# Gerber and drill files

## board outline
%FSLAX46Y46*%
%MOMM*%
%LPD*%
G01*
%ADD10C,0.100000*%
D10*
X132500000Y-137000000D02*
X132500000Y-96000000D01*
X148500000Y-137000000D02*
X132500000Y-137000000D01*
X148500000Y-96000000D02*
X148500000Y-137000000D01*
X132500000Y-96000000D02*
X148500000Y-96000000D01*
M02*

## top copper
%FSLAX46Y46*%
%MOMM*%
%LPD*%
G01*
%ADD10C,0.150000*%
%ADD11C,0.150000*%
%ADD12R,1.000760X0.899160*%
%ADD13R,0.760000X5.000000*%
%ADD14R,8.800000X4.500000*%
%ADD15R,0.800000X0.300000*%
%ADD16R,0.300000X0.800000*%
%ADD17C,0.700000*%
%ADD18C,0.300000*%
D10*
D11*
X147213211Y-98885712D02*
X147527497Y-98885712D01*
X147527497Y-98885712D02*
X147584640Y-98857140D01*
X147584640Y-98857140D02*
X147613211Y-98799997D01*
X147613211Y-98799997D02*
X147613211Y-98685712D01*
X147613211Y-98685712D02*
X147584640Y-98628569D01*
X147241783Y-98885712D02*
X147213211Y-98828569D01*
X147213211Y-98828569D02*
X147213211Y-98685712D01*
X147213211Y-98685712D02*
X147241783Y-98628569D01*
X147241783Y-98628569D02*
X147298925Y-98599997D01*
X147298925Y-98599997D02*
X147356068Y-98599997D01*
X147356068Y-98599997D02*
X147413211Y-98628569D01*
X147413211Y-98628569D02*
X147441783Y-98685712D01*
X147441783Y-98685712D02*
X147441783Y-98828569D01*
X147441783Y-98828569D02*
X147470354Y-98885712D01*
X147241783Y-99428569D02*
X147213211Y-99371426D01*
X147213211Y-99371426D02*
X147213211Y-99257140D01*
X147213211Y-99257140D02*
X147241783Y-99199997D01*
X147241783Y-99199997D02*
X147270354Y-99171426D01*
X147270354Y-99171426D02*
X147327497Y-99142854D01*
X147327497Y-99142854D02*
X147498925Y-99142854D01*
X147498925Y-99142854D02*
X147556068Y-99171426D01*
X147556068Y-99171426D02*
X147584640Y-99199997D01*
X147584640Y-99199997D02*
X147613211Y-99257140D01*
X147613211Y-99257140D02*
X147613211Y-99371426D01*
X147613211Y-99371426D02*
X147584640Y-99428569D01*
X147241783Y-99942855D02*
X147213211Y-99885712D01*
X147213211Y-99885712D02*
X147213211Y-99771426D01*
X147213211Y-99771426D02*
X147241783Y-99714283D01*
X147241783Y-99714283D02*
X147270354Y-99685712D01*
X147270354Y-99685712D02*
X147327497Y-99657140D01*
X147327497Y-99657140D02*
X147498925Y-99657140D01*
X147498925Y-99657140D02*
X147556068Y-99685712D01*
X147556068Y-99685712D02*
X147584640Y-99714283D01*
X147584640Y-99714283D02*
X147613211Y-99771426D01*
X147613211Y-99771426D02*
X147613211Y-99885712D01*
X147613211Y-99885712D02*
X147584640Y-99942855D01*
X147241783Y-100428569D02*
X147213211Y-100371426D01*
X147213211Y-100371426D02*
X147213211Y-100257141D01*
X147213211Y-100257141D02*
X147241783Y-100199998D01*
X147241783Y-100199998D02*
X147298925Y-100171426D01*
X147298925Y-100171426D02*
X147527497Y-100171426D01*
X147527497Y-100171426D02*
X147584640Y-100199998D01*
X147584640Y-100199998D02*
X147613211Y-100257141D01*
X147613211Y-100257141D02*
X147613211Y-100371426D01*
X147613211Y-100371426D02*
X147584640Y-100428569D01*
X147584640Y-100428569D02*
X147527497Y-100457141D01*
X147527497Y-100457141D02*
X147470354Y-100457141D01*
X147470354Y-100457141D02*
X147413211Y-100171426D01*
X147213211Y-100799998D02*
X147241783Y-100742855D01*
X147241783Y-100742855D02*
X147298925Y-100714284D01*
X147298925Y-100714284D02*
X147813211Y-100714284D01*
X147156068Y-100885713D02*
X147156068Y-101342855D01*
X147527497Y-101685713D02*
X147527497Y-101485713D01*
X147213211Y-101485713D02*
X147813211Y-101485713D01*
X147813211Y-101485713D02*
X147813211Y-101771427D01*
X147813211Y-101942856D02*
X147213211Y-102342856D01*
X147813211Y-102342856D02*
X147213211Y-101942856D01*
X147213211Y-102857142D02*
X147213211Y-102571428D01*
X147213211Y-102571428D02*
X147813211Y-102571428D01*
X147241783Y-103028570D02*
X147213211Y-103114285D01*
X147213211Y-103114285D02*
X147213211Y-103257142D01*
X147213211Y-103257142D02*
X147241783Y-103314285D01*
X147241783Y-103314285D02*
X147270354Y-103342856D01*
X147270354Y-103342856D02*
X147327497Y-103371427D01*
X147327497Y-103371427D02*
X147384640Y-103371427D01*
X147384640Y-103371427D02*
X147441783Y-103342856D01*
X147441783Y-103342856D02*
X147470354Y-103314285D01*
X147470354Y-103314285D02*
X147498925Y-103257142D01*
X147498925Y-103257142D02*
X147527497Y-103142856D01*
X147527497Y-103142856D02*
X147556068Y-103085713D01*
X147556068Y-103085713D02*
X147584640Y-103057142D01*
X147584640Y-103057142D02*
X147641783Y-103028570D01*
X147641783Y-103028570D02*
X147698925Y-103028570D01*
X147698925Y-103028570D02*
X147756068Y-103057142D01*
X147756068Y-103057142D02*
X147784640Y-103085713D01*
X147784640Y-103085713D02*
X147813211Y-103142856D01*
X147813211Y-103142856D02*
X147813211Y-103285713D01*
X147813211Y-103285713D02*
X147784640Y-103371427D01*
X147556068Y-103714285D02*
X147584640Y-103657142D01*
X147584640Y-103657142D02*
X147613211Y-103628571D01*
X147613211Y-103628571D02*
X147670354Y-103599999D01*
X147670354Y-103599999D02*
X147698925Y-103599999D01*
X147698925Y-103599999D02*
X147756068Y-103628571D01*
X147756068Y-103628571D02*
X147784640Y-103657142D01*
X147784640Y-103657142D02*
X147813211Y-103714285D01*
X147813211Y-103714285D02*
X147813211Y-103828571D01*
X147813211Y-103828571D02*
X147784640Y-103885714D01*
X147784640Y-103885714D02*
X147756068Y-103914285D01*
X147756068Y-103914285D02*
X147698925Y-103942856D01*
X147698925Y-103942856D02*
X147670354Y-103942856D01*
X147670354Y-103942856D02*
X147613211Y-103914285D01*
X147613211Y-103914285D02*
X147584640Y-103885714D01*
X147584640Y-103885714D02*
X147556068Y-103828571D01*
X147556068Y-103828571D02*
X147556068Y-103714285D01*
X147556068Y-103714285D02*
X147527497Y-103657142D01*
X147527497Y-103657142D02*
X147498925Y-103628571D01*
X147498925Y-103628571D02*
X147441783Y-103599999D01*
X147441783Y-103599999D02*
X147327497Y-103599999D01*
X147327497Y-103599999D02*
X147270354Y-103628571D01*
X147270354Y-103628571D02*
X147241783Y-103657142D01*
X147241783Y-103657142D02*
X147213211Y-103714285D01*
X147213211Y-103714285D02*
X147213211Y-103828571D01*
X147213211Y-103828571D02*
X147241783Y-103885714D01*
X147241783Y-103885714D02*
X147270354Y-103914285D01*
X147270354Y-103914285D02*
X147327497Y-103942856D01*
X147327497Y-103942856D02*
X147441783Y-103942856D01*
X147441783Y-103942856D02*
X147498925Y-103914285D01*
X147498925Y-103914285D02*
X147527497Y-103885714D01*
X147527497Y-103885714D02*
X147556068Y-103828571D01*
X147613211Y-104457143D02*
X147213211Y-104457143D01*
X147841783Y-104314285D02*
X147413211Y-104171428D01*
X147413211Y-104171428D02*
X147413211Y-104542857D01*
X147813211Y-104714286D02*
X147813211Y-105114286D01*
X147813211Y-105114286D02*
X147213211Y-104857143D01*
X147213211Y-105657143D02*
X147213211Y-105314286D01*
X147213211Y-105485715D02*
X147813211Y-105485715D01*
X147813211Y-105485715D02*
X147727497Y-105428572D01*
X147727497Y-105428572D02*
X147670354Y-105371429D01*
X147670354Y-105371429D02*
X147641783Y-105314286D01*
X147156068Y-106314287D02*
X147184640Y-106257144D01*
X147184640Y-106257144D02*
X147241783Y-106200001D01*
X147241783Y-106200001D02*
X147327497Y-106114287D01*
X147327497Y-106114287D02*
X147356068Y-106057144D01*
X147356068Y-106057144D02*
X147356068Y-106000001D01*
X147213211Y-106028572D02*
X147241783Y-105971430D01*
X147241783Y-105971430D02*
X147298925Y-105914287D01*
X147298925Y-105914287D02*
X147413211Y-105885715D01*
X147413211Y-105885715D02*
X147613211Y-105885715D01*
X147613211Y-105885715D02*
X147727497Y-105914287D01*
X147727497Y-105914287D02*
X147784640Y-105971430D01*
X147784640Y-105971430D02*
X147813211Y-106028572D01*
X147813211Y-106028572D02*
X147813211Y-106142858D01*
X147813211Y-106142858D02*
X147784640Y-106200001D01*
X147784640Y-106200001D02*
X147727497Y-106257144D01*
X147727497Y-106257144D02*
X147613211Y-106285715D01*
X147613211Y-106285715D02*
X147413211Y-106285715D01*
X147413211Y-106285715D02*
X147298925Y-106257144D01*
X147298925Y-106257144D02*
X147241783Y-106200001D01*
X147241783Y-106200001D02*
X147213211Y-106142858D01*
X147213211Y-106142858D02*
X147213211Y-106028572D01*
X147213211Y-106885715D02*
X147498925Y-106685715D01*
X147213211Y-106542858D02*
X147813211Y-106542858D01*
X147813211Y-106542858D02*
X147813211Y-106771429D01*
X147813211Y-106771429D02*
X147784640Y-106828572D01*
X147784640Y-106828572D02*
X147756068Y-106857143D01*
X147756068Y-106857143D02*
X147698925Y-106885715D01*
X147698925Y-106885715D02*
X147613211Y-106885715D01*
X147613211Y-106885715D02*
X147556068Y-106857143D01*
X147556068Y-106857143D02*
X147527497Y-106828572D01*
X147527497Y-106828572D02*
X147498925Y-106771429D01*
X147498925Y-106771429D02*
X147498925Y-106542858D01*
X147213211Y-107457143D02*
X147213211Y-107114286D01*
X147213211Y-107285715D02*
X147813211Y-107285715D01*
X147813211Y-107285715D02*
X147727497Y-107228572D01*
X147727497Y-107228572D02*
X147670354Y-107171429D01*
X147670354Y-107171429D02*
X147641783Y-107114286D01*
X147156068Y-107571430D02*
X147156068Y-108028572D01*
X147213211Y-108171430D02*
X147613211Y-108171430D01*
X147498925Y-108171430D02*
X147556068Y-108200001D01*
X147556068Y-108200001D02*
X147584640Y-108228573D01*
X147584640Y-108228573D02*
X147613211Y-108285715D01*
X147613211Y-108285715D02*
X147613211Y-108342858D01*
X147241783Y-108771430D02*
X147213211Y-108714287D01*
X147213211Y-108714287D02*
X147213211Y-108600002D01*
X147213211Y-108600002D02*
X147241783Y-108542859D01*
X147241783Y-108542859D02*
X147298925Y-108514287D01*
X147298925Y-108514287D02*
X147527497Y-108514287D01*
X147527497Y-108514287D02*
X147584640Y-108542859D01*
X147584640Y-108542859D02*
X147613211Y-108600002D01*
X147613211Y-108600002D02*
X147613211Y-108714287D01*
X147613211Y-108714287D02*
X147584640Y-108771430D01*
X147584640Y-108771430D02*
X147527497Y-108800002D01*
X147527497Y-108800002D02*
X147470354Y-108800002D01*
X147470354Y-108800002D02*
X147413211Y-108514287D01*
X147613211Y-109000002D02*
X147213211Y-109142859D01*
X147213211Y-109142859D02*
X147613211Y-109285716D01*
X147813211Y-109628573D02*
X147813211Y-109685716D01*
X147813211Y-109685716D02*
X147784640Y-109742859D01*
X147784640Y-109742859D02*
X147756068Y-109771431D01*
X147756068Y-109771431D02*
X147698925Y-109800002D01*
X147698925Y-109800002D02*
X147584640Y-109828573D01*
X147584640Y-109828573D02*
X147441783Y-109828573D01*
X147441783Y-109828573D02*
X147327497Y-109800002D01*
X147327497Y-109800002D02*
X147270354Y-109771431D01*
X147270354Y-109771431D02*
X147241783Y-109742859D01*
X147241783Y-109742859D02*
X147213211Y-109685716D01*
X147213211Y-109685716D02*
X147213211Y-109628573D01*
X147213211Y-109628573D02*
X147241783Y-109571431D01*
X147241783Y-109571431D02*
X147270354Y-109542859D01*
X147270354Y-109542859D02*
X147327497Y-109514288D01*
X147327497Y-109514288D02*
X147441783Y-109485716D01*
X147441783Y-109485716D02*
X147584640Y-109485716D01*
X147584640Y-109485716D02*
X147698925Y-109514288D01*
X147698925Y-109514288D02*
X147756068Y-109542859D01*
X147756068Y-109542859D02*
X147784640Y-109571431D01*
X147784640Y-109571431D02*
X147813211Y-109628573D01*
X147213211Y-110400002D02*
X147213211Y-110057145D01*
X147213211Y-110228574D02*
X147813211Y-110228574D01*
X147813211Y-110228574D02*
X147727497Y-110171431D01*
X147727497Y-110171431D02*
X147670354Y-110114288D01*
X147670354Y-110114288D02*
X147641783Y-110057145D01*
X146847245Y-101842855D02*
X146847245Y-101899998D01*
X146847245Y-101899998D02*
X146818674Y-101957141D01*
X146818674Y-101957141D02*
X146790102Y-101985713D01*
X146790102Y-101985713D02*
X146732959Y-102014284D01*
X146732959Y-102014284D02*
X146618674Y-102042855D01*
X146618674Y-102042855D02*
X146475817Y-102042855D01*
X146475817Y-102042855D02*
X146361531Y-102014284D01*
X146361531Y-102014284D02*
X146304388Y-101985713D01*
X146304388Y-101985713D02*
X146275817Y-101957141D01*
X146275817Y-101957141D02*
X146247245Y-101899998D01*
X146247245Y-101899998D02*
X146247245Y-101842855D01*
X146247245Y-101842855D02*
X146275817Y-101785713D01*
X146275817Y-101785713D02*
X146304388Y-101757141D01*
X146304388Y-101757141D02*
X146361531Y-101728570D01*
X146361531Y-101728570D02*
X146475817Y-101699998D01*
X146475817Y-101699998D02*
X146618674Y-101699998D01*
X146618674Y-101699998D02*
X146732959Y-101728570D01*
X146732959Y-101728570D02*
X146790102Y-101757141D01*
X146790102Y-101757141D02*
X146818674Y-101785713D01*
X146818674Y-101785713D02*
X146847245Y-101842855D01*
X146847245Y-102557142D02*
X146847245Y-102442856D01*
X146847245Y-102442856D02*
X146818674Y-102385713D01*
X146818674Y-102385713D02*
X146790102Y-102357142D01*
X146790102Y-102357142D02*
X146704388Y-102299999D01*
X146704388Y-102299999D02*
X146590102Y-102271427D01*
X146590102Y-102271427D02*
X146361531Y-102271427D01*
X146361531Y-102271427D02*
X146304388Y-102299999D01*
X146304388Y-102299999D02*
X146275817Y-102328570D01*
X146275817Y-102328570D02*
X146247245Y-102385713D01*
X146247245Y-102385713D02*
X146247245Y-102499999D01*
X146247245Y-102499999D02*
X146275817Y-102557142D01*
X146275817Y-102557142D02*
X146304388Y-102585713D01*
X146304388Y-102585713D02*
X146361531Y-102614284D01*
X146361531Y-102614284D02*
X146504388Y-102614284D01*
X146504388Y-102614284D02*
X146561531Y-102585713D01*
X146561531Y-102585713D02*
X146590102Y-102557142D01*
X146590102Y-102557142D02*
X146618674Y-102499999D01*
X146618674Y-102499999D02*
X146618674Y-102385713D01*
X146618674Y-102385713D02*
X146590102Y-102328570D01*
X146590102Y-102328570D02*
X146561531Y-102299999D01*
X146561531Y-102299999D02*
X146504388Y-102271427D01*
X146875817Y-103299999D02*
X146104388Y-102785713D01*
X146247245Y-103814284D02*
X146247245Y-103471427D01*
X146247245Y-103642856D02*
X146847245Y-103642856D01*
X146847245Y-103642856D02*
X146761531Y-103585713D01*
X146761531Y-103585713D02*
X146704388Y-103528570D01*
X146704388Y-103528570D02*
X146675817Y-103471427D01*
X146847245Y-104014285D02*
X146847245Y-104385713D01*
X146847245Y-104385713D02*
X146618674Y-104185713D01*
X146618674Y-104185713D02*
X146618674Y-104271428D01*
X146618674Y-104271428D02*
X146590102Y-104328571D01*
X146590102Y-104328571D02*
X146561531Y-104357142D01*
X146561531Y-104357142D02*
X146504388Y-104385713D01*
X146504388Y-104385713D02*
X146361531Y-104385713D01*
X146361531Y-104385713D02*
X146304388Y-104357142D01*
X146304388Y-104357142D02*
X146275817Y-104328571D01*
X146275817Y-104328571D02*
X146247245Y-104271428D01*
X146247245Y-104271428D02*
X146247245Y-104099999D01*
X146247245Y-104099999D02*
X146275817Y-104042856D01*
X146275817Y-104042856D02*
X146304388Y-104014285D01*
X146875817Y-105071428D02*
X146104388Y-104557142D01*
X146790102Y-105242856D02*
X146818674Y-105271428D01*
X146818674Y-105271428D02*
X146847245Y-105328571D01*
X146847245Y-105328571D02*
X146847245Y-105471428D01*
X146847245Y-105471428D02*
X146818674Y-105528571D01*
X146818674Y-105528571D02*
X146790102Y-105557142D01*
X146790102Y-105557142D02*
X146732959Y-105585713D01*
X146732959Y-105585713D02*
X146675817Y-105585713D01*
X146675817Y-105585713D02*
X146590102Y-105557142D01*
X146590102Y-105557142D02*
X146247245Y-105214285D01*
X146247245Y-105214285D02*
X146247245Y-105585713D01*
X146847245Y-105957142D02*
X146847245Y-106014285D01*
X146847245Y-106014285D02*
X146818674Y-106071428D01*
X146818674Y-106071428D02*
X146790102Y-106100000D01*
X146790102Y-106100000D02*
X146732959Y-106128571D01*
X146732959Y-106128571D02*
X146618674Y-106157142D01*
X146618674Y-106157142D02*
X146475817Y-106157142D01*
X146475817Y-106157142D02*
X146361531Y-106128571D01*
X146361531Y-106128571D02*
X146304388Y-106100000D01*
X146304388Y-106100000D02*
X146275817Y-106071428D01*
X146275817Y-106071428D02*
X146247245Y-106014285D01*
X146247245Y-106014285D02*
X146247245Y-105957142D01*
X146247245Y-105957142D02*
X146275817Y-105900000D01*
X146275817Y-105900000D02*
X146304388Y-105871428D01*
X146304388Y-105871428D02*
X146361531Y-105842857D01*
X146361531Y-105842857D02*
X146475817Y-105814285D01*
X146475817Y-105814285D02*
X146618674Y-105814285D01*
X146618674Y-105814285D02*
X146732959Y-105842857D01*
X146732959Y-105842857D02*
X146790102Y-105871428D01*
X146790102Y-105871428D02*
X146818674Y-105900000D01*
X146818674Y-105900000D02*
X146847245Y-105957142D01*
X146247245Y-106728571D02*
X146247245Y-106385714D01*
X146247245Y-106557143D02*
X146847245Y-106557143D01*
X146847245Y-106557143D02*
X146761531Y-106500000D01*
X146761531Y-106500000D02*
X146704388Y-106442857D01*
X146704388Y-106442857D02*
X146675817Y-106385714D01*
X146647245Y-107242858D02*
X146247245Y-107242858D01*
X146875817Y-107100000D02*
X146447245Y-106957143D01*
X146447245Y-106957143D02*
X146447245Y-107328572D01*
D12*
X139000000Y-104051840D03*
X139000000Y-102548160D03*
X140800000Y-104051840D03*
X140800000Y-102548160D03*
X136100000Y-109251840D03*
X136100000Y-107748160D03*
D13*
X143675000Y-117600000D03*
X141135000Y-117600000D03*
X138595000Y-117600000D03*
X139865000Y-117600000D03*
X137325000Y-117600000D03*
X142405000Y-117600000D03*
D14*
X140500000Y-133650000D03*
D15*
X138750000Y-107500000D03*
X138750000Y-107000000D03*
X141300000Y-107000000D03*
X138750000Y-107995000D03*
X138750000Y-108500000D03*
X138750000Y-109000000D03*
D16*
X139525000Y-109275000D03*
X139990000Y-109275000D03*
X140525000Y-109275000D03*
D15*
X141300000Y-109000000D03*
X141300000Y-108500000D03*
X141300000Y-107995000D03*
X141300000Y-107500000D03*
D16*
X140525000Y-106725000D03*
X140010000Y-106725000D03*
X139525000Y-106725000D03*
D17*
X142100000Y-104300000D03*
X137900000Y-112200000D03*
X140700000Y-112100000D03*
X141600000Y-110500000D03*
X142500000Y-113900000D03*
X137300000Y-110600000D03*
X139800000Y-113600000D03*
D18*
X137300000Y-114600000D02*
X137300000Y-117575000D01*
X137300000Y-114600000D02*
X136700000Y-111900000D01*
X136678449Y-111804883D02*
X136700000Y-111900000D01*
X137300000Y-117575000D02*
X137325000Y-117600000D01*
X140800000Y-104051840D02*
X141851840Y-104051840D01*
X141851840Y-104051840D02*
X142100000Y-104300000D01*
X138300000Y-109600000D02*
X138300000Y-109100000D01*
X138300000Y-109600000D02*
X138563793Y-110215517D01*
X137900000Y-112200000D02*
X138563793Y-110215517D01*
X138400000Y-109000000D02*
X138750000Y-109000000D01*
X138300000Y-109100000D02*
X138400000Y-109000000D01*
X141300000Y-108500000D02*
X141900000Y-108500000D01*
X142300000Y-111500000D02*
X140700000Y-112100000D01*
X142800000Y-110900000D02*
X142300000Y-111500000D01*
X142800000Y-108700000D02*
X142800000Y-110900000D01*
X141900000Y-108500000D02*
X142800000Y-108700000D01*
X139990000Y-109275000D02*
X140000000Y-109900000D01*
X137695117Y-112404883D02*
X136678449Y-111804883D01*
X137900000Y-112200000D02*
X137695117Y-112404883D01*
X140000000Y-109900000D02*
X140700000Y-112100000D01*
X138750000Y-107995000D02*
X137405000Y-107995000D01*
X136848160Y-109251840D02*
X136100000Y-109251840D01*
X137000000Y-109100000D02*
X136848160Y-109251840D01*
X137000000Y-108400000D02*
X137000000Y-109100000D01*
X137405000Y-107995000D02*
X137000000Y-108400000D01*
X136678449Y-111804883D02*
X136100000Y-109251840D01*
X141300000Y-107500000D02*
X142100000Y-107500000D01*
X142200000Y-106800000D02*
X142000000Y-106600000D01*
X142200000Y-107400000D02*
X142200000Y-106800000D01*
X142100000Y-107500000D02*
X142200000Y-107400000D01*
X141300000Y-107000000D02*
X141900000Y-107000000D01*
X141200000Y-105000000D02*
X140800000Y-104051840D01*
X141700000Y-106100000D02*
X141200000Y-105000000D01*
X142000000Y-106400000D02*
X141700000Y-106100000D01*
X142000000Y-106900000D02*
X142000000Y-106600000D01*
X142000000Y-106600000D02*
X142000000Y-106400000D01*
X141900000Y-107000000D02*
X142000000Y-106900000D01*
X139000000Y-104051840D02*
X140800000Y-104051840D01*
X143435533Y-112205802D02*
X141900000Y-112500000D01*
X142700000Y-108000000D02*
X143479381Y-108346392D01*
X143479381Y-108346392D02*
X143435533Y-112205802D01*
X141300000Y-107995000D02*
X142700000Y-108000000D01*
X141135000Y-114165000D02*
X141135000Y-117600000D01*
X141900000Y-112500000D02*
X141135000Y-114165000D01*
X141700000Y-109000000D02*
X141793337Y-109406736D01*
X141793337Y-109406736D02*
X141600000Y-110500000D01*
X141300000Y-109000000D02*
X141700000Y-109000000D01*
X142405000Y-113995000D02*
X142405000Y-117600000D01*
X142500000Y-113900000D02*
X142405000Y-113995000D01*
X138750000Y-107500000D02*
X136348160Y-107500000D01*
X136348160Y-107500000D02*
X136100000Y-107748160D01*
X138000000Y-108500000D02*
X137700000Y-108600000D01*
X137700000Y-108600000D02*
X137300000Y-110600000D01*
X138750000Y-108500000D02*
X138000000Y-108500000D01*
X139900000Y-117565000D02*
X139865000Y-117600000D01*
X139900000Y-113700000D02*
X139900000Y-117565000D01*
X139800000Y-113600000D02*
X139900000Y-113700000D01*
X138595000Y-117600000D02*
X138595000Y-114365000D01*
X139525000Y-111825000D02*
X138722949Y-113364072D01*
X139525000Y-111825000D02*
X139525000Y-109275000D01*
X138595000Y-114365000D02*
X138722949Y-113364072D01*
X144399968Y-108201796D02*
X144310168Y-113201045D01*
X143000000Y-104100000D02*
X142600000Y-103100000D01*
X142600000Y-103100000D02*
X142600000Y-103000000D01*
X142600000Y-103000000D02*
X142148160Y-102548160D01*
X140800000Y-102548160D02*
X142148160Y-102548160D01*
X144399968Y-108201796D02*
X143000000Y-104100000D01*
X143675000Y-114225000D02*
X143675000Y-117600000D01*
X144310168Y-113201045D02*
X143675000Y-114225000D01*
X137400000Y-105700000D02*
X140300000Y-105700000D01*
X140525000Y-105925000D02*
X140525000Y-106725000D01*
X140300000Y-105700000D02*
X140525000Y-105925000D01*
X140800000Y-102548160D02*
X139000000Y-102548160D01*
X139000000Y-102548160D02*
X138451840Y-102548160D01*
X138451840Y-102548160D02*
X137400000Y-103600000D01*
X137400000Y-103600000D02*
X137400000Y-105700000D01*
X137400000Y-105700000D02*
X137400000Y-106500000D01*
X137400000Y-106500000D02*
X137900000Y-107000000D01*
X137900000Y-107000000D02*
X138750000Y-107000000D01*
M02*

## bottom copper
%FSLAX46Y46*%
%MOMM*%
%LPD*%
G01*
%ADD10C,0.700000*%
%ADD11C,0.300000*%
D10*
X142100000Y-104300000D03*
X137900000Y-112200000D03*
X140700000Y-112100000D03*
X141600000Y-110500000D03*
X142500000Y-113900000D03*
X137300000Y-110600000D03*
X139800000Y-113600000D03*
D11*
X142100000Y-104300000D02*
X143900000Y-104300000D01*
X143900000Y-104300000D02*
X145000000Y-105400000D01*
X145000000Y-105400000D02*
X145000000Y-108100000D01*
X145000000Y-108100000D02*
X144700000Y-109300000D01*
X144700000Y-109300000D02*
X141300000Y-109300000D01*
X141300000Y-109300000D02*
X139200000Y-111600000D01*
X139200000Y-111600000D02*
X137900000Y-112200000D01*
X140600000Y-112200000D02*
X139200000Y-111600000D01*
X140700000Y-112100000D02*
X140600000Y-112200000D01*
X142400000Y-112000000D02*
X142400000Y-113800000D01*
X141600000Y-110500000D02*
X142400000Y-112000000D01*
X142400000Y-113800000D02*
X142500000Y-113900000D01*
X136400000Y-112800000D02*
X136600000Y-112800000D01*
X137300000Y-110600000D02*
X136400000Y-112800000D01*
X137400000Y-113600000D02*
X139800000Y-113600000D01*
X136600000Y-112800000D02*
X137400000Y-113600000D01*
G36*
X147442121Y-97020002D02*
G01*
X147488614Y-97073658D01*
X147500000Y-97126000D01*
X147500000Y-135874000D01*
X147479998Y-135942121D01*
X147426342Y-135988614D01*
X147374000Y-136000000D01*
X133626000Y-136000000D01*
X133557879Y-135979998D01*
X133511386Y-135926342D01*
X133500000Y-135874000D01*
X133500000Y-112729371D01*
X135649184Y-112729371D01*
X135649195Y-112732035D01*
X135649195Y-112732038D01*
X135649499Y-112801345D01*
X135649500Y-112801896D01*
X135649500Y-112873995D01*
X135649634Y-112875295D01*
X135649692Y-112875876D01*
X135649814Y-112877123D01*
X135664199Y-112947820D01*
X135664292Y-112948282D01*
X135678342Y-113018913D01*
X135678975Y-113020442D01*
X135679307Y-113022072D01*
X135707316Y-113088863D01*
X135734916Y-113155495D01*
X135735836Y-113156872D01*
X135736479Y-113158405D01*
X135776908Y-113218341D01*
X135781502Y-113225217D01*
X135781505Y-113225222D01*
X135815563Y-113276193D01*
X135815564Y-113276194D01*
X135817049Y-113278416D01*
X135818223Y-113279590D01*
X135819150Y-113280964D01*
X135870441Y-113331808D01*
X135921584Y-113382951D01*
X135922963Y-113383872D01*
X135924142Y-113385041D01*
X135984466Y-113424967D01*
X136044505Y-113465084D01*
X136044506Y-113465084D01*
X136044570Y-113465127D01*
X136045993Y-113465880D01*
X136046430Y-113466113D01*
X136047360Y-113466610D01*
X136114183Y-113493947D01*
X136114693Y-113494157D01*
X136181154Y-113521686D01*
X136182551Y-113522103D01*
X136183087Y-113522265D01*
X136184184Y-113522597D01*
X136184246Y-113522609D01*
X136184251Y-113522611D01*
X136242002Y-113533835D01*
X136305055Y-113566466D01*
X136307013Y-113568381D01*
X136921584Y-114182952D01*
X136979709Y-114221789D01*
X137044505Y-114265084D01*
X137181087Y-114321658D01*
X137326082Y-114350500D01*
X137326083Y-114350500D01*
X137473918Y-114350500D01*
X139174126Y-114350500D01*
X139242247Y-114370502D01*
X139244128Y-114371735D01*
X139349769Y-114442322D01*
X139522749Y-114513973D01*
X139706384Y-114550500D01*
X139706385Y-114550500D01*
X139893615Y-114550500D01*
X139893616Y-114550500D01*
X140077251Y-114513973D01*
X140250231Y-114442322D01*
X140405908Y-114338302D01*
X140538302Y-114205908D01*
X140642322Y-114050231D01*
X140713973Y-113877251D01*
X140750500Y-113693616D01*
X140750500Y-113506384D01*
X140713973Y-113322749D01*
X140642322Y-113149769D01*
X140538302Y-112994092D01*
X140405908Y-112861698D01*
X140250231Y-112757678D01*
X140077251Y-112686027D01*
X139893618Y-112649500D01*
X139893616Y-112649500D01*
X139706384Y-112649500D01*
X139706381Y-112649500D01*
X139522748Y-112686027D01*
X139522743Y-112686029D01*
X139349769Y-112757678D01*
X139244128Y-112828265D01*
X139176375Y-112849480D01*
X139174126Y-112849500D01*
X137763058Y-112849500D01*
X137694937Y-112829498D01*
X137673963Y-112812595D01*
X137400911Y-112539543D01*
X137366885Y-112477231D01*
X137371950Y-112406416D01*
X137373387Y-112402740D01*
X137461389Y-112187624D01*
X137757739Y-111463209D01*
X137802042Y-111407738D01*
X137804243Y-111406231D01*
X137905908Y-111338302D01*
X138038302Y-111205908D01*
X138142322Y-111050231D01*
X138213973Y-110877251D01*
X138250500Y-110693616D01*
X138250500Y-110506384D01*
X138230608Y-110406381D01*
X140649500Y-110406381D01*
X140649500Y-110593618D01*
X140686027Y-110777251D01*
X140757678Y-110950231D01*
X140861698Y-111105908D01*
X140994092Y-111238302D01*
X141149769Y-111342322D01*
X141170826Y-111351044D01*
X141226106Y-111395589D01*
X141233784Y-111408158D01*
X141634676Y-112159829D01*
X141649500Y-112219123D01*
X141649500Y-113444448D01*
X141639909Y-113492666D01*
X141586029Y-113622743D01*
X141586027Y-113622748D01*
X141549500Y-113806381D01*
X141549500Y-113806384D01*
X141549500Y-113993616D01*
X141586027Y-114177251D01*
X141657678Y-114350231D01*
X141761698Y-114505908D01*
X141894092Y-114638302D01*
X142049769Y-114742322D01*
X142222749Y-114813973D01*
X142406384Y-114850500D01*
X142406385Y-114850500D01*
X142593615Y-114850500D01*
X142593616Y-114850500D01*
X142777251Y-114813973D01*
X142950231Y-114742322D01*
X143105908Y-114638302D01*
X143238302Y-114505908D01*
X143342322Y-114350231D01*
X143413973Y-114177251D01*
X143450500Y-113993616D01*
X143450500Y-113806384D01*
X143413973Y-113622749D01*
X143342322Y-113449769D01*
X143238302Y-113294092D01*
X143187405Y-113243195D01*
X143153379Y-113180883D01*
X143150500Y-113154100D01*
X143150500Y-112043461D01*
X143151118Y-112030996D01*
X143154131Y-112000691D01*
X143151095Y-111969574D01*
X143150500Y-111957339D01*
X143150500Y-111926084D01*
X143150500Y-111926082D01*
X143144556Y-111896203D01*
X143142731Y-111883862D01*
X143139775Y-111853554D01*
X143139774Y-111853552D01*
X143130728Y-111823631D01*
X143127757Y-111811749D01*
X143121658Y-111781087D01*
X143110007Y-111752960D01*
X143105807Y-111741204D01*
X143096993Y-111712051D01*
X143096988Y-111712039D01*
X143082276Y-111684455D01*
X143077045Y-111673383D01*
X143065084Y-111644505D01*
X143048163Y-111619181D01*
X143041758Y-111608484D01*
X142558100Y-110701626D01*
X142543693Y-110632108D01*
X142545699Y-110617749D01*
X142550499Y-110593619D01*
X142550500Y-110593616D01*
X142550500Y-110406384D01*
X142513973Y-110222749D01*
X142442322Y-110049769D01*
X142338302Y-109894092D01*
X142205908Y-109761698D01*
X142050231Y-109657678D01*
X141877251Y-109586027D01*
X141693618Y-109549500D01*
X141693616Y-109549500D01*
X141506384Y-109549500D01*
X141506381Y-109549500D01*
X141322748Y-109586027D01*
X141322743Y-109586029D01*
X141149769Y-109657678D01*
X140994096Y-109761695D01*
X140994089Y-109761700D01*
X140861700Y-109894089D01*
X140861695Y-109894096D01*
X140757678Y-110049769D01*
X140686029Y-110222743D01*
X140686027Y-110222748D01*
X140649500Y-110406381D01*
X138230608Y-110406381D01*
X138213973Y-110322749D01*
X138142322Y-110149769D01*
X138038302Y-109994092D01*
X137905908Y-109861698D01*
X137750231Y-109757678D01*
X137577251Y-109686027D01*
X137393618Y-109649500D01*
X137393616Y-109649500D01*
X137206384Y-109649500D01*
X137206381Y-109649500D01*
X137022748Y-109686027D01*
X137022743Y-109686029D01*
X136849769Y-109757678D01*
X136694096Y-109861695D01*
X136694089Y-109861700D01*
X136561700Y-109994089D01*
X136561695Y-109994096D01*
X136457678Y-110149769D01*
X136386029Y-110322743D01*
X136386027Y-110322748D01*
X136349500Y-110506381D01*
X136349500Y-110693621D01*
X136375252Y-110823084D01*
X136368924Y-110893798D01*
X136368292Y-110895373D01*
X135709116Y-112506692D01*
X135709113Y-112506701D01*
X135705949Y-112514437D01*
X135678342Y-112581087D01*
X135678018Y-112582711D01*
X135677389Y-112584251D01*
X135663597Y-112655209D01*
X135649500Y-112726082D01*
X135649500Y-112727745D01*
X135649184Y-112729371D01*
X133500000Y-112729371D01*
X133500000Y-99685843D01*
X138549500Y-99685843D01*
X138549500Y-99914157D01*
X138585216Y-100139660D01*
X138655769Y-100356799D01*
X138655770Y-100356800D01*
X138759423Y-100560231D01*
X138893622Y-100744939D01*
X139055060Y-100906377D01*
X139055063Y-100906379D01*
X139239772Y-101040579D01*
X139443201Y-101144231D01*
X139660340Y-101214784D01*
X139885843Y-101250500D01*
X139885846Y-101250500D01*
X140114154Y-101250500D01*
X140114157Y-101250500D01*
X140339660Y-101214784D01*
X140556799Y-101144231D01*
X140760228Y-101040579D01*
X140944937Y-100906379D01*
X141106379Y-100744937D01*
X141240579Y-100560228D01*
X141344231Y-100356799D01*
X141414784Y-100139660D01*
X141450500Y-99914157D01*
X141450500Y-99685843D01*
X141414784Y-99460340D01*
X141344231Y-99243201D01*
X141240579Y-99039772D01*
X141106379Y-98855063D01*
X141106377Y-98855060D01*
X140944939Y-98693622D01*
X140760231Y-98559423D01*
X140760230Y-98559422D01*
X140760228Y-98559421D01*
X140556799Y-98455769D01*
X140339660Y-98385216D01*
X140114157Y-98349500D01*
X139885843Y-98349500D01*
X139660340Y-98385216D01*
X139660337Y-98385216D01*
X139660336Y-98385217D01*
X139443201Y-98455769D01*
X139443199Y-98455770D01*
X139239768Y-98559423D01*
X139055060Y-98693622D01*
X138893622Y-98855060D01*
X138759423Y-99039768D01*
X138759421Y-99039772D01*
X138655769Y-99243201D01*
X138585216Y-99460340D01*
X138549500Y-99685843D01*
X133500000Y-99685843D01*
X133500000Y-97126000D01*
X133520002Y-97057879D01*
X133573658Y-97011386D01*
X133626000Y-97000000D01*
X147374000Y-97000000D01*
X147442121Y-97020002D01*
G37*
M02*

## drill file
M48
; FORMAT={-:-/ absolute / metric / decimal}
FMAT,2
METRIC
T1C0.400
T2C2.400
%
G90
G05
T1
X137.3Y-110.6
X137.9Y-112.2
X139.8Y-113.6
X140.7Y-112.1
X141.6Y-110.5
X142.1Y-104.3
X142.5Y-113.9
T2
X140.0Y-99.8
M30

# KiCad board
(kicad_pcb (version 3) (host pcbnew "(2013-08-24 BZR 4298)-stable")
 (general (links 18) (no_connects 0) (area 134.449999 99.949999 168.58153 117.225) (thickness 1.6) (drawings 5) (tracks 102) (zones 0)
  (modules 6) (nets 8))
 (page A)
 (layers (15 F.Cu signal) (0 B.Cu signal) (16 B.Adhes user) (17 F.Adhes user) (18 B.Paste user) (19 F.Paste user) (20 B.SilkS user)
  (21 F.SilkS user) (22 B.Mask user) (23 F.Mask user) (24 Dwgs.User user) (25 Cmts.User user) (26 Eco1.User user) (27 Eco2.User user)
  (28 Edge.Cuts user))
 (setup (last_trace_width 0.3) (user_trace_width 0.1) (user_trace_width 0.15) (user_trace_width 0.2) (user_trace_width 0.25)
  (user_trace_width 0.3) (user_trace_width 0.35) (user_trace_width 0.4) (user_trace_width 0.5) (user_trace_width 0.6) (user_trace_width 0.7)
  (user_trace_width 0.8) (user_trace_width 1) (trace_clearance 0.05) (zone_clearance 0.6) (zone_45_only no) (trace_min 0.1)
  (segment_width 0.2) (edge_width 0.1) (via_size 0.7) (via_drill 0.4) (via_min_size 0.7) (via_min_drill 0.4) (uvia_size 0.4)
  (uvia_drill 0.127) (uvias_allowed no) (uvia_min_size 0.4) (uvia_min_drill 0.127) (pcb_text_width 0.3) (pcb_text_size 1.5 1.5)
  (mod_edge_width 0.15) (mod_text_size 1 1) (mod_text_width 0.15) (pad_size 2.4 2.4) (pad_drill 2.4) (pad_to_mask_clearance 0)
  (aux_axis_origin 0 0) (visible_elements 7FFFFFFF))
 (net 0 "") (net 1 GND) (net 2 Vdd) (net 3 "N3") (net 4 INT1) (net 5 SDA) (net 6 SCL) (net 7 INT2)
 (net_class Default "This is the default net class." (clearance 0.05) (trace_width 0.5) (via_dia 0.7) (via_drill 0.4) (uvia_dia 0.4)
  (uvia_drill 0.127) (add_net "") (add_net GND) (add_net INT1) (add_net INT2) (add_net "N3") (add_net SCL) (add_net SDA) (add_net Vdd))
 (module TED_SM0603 (layer F.Cu) (at 139 103.3 270)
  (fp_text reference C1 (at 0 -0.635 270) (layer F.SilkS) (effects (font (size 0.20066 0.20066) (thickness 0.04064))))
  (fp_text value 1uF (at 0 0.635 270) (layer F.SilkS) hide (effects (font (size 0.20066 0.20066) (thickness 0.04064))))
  (pad 2 smd rect (at 0.75184 0 270) (size 0.89916 1.00076) (layers F.Cu F.Paste F.Mask) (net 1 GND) (clearance 0.1))
  (pad 1 smd rect (at -0.75184 0 270) (size 0.89916 1.00076) (layers F.Cu F.Paste F.Mask) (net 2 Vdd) (clearance 0.1)))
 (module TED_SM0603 (layer F.Cu) (at 140.8 103.3 270)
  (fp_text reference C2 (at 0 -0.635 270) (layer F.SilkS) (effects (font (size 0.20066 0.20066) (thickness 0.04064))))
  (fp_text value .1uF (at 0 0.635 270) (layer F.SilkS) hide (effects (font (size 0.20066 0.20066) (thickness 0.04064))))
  (pad 2 smd rect (at 0.75184 0 270) (size 0.89916 1.00076) (layers F.Cu F.Paste F.Mask) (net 1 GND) (clearance 0.1))
  (pad 1 smd rect (at -0.75184 0 270) (size 0.89916 1.00076) (layers F.Cu F.Paste F.Mask) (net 2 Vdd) (clearance 0.1)))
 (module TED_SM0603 (layer F.Cu) (at 136.1 108.5 270)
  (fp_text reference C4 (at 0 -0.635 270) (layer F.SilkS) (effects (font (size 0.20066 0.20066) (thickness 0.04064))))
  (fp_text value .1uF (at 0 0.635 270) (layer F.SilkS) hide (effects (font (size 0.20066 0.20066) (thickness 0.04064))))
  (pad 2 smd rect (at 0.75184 0 270) (size 0.89916 1.00076) (layers F.Cu F.Paste F.Mask) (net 1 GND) (clearance 0.1))
  (pad 1 smd rect (at -0.75184 0 270) (size 0.89916 1.00076) (layers F.Cu F.Paste F.Mask) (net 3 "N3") (clearance 0.1)))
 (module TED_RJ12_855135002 (layer F.Cu) (at 140.5 125.5 180)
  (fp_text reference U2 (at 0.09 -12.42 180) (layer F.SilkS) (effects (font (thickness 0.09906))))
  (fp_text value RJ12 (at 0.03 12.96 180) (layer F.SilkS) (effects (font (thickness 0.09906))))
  (pad 6 smd rect (at -3.175 7.9 180) (size 0.76 5) (layers F.Cu F.Paste F.Mask) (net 2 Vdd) (clearance 0.2))
  (pad 4 smd rect (at -0.635 7.9 180) (size 0.76 5) (layers F.Cu F.Paste F.Mask) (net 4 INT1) (clearance 0.2))
  (pad 2 smd rect (at 1.905 7.9 180) (size 0.76 5) (layers F.Cu F.Paste F.Mask) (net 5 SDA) (clearance 0.2))
  (pad 3 smd rect (at 0.635 7.9 180) (size 0.76 5) (layers F.Cu F.Paste F.Mask) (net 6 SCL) (clearance 0.2))
  (pad 1 smd rect (at 3.175 7.9 180) (size 0.76 5) (layers F.Cu F.Paste F.Mask) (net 1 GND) (clearance 0.2))
  (pad 5 smd rect (at -1.905 7.9 180) (size 0.76 5) (layers F.Cu F.Paste F.Mask) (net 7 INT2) (clearance 0.2))
  (pad PAD smd rect (at 0 -8.15 180) (size 8.8 4.5) (layers F.Cu F.Paste F.Mask)))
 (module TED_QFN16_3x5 (layer F.Cu) (at 140.025 108) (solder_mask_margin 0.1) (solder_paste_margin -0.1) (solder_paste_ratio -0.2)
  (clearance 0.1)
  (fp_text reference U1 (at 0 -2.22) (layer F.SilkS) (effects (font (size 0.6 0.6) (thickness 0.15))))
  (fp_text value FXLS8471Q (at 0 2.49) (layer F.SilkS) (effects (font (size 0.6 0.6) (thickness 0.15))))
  (pad 2 smd rect (at -1.275 -0.5) (size 0.8 0.3) (layers F.Cu F.Paste F.Mask) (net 3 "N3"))
  (pad 1 smd rect (at -1.275 -1) (size 0.8 0.3) (layers F.Cu F.Paste F.Mask) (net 2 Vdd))
  (pad 13 smd rect (at 1.275 -1) (size 0.8 0.3) (layers F.Cu F.Paste F.Mask) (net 1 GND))
  (pad 3 smd rect (at -1.275 -0.005) (size 0.8 0.3) (layers F.Cu F.Paste F.Mask) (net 1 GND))
  (pad 4 smd rect (at -1.275 0.5) (size 0.8 0.3) (layers F.Cu F.Paste F.Mask) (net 6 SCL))
  (pad 5 smd rect (at -1.275 1) (size 0.8 0.3) (layers F.Cu F.Paste F.Mask) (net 1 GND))
  (pad 6 smd rect (at -0.5 1.275) (size 0.3 0.8) (layers F.Cu F.Paste F.Mask) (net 5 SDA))
  (pad 7 smd rect (at -0.035 1.275) (size 0.3 0.8) (layers F.Cu F.Paste F.Mask) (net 1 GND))
  (pad 8 smd rect (at 0.5 1.275) (size 0.3 0.8) (layers F.Cu F.Paste F.Mask))
  (pad 9 smd rect (at 1.275 1) (size 0.8 0.3) (layers F.Cu F.Paste F.Mask) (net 7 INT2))
  (pad 10 smd rect (at 1.275 0.5) (size 0.8 0.3) (layers F.Cu F.Paste F.Mask) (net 1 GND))
  (pad 11 smd rect (at 1.275 -0.005) (size 0.8 0.3) (layers F.Cu F.Paste F.Mask) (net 4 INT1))
  (pad 12 smd rect (at 1.275 -0.5) (size 0.8 0.3) (layers F.Cu F.Paste F.Mask) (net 1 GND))
  (pad 14 smd rect (at 0.5 -1.275) (size 0.3 0.8) (layers F.Cu F.Paste F.Mask) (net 2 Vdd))
  (pad 15 smd rect (at -0.015 -1.275) (size 0.3 0.8) (layers F.Cu F.Paste F.Mask))
  (pad 16 smd rect (at -0.5 -1.275) (size 0.3 0.8) (layers F.Cu F.Paste F.Mask)))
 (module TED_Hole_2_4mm (layer F.Cu) (at 140 99.8)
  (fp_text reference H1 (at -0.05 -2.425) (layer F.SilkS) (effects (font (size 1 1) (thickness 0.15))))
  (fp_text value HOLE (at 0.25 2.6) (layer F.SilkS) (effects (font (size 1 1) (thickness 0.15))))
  (pad "" np_thru_hole circle (at 0 0) (size 2.4 2.4) (drill 2.4) (layers *.Cu *.Mask F.SilkS)))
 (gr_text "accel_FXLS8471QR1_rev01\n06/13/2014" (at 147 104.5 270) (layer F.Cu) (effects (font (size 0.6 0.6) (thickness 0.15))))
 (gr_line (start 132.5 137) (end 132.5 96) (angle 90) (layer Edge.Cuts) (width 0.1))
 (gr_line (start 148.5 137) (end 132.5 137) (angle 90) (layer Edge.Cuts) (width 0.1))
 (gr_line (start 148.5 96) (end 148.5 137) (angle 90) (layer Edge.Cuts) (width 0.1))
 (gr_line (start 132.5 96) (end 148.5 96) (angle 90) (layer Edge.Cuts) (width 0.1))
 (segment (start 137.3 114.6) (end 137.3 117.575) (width 0.3) (layer F.Cu) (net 1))
 (segment (start 137.3 114.6) (end 136.7 111.9) (width 0.3) (layer F.Cu) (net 1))
 (segment (start 136.678449 111.804883) (end 136.7 111.9) (width 0.3) (layer F.Cu) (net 1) (status 20))
 (segment (start 137.3 117.575) (end 137.325 117.6) (width 0.3) (layer F.Cu) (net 1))
 (segment (start 140.8 104.05184) (end 141.85184 104.05184) (width 0.3) (layer F.Cu) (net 1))
 (segment (start 141.85184 104.05184) (end 142.1 104.3) (width 0.3) (layer F.Cu) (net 1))
 (via (at 142.1 104.3) (size 0.7) (layers F.Cu B.Cu) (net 1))
 (segment (start 142.1 104.3) (end 143.9 104.3) (width 0.3) (layer B.Cu) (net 1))
 (segment (start 143.9 104.3) (end 145 105.4) (width 0.3) (layer B.Cu) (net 1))
 (segment (start 145 105.4) (end 145 108.1) (width 0.3) (layer B.Cu) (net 1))
 (segment (start 145 108.1) (end 144.7 109.3) (width 0.3) (layer B.Cu) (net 1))
 (segment (start 144.7 109.3) (end 141.3 109.3) (width 0.3) (layer B.Cu) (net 1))
 (segment (start 141.3 109.3) (end 139.2 111.6) (width 0.3) (layer B.Cu) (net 1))
 (segment (start 138.3 109.6) (end 138.3 109.1) (width 0.3) (layer F.Cu) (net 1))
 (segment (start 138.3 109.6) (end 138.563793 110.215517) (width 0.3) (layer F.Cu) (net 1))
 (segment (start 137.9 112.2) (end 138.563793 110.215517) (width 0.3) (layer F.Cu) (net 1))
 (segment (start 138.4 109) (end 138.75 109) (width 0.3) (layer F.Cu) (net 1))
 (segment (start 138.3 109.1) (end 138.4 109) (width 0.3) (layer F.Cu) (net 1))
 (segment (start 141.3 108.5) (end 141.9 108.5) (width 0.3) (layer F.Cu) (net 1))
 (segment (start 142.3 111.5) (end 140.7 112.1) (width 0.3) (layer F.Cu) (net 1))
 (segment (start 142.8 110.9) (end 142.3 111.5) (width 0.3) (layer F.Cu) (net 1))
 (segment (start 142.8 108.7) (end 142.8 110.9) (width 0.3) (layer F.Cu) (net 1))
 (segment (start 141.9 108.5) (end 142.8 108.7) (width 0.3) (layer F.Cu) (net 1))
 (segment (start 139.99 109.275) (end 140 109.9) (width 0.3) (layer F.Cu) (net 1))
 (segment (start 137.695117 112.404883) (end 136.678449 111.804883) (width 0.3) (layer F.Cu) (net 1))
 (segment (start 137.9 112.2) (end 137.695117 112.404883) (width 0.3) (layer F.Cu) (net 1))
 (via (at 137.9 112.2) (size 0.7) (layers F.Cu B.Cu) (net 1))
 (segment (start 139.2 111.6) (end 137.9 112.2) (width 0.3) (layer B.Cu) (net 1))
 (segment (start 140.6 112.2) (end 139.2 111.6) (width 0.3) (layer B.Cu) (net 1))
 (via (at 140.7 112.1) (size 0.7) (layers F.Cu B.Cu) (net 1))
 (segment (start 140.7 112.1) (end 140.6 112.2) (width 0.3) (layer B.Cu) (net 1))
 (segment (start 140 109.9) (end 140.7 112.1) (width 0.3) (layer F.Cu) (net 1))
 (segment (start 138.75 107.995) (end 137.405 107.995) (width 0.3) (layer F.Cu) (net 1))
 (segment (start 136.84816 109.25184) (end 136.1 109.25184) (width 0.3) (layer F.Cu) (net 1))
 (segment (start 137 109.1) (end 136.84816 109.25184) (width 0.3) (layer F.Cu) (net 1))
 (segment (start 137 108.4) (end 137 109.1) (width 0.3) (layer F.Cu) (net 1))
 (segment (start 137.405 107.995) (end 137 108.4) (width 0.3) (layer F.Cu) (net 1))
 (segment (start 136.678449 111.804883) (end 136.1 109.25184) (width 0.3) (layer F.Cu) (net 1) (status 20))
 (segment (start 141.3 107.5) (end 142.1 107.5) (width 0.3) (layer F.Cu) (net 1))
 (segment (start 142.2 106.8) (end 142 106.6) (width 0.3) (layer F.Cu) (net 1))
 (segment (start 142.2 107.4) (end 142.2 106.8) (width 0.3) (layer F.Cu) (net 1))
 (segment (start 142.1 107.5) (end 142.2 107.4) (width 0.3) (layer F.Cu) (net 1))
 (segment (start 141.3 107) (end 141.9 107) (width 0.3) (layer F.Cu) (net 1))
 (segment (start 141.2 105) (end 140.8 104.05184) (width 0.3) (layer F.Cu) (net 1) (status 20))
 (segment (start 141.7 106.1) (end 141.2 105) (width 0.3) (layer F.Cu) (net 1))
 (segment (start 142 106.4) (end 141.7 106.1) (width 0.3) (layer F.Cu) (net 1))
 (segment (start 142 106.9) (end 142 106.6) (width 0.3) (layer F.Cu) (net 1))
 (segment (start 142 106.6) (end 142 106.4) (width 0.3) (layer F.Cu) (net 1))
 (segment (start 141.9 107) (end 142 106.9) (width 0.3) (layer F.Cu) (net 1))
 (segment (start 139 104.05184) (end 140.8 104.05184) (width 0.3) (layer F.Cu) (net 1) (status 20))
 (segment (start 143.435533 112.205802) (end 141.9 112.5) (width 0.3) (layer F.Cu) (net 4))
 (segment (start 142.7 108) (end 143.479381 108.346392) (width 0.3) (layer F.Cu) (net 4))
 (segment (start 143.479381 108.346392) (end 143.435533 112.205802) (width 0.3) (layer F.Cu) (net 4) (status 20))
 (segment (start 141.3 107.995) (end 142.7 108) (width 0.3) (layer F.Cu) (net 4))
 (segment (start 141.135 114.165) (end 141.135 117.6) (width 0.3) (layer F.Cu) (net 4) (status 800000))
 (segment (start 141.9 112.5) (end 141.135 114.165) (width 0.3) (layer F.Cu) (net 4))
 (segment (start 142.4 112) (end 142.4 113.8) (width 0.3) (layer B.Cu) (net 7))
 (segment (start 141.7 109) (end 141.793337 109.406736) (width 0.3) (layer F.Cu) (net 7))
 (segment (start 141.793337 109.406736) (end 141.6 110.5) (width 0.3) (layer F.Cu) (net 7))
 (via (at 141.6 110.5) (size 0.7) (layers F.Cu B.Cu) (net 7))
 (segment (start 141.6 110.5) (end 142.4 112) (width 0.3) (layer B.Cu) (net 7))
 (segment (start 141.3 109) (end 141.7 109) (width 0.3) (layer F.Cu) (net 7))
 (segment (start 142.405 113.995) (end 142.405 117.6) (width 0.3) (layer F.Cu) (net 7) (status 800000))
 (segment (start 142.5 113.9) (end 142.405 113.995) (width 0.3) (layer F.Cu) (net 7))
 (via (at 142.5 113.9) (size 0.7) (layers F.Cu B.Cu) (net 7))
 (segment (start 142.4 113.8) (end 142.5 113.9) (width 0.3) (layer B.Cu) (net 7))
 (segment (start 138.75 107.5) (end 136.34816 107.5) (width 0.3) (layer F.Cu) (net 3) (status 20))
 (segment (start 136.34816 107.5) (end 136.1 107.74816) (width 0.3) (layer F.Cu) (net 3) (status 30))
 (segment (start 136.4 112.8) (end 136.6 112.8) (width 0.3) (layer B.Cu) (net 6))
 (segment (start 138 108.5) (end 137.7 108.6) (width 0.3) (layer F.Cu) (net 6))
 (segment (start 137.7 108.6) (end 137.3 110.6) (width 0.3) (layer F.Cu) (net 6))
 (via (at 137.3 110.6) (size 0.7) (layers F.Cu B.Cu) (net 6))
 (segment (start 137.3 110.6) (end 136.4 112.8) (width 0.3) (layer B.Cu) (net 6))
 (segment (start 138.75 108.5) (end 138 108.5) (width 0.3) (layer F.Cu) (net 6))
 (segment (start 139.9 117.565) (end 139.865 117.6) (width 0.3) (layer F.Cu) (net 6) (status C00000))
 (segment (start 139.9 113.7) (end 139.9 117.565) (width 0.3) (layer F.Cu) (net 6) (status 800000))
 (segment (start 139.8 113.6) (end 139.9 113.7) (width 0.3) (layer F.Cu) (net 6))
 (via (at 139.8 113.6) (size 0.7) (layers F.Cu B.Cu) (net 6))
 (segment (start 137.4 113.6) (end 139.8 113.6) (width 0.3) (layer B.Cu) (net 6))
 (segment (start 136.6 112.8) (end 137.4 113.6) (width 0.3) (layer B.Cu) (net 6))
 (segment (start 138.595 117.6) (end 138.595 114.365) (width 0.3) (layer F.Cu) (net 5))
 (segment (start 139.525 111.825) (end 138.722949 113.364072) (width 0.3) (layer F.Cu) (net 5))
 (segment (start 139.525 111.825) (end 139.525 109.275) (width 0.3) (layer F.Cu) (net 5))
 (segment (start 138.595 114.365) (end 138.722949 113.364072) (width 0.3) (layer F.Cu) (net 5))
 (segment (start 144.399968 108.201796) (end 144.310168 113.201045) (width 0.3) (layer F.Cu) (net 2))
 (segment (start 143 104.1) (end 142.6 103.1) (width 0.3) (layer F.Cu) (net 2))
 (segment (start 142.6 103.1) (end 142.6 103) (width 0.3) (layer F.Cu) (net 2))
 (segment (start 142.6 103) (end 142.14816 102.54816) (width 0.3) (layer F.Cu) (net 2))
 (segment (start 140.8 102.54816) (end 142.14816 102.54816) (width 0.3) (layer F.Cu) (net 2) (status 20))
 (segment (start 144.399968 108.201796) (end 143 104.1) (width 0.3) (layer F.Cu) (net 2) (status 10))
 (segment (start 143.675 114.225) (end 143.675 117.6) (width 0.3) (layer F.Cu) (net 2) (status 800000))
 (segment (start 144.310168 113.201045) (end 143.675 114.225) (width 0.3) (layer F.Cu) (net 2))
 (segment (start 137.4 105.7) (end 140.3 105.7) (width 0.3) (layer F.Cu) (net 2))
 (segment (start 140.525 105.925) (end 140.525 106.725) (width 0.3) (layer F.Cu) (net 2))
 (segment (start 140.3 105.7) (end 140.525 105.925) (width 0.3) (layer F.Cu) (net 2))
 (segment (start 140.8 102.54816) (end 139 102.54816) (width 0.3) (layer F.Cu) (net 2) (status 10))
 (segment (start 139 102.54816) (end 138.45184 102.54816) (width 0.3) (layer F.Cu) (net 2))
 (segment (start 138.45184 102.54816) (end 137.4 103.6) (width 0.3) (layer F.Cu) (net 2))
 (segment (start 137.4 103.6) (end 137.4 105.7) (width 0.3) (layer F.Cu) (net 2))
 (segment (start 137.4 105.7) (end 137.4 106.5) (width 0.3) (layer F.Cu) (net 2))
 (segment (start 137.4 106.5) (end 137.9 107) (width 0.3) (layer F.Cu) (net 2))
 (segment (start 137.9 107) (end 138.75 107) (width 0.3) (layer F.Cu) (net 2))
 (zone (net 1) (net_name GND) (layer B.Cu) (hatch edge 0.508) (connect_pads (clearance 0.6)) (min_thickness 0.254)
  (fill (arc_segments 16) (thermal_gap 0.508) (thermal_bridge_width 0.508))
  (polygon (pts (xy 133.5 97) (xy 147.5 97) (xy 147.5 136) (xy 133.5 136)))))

